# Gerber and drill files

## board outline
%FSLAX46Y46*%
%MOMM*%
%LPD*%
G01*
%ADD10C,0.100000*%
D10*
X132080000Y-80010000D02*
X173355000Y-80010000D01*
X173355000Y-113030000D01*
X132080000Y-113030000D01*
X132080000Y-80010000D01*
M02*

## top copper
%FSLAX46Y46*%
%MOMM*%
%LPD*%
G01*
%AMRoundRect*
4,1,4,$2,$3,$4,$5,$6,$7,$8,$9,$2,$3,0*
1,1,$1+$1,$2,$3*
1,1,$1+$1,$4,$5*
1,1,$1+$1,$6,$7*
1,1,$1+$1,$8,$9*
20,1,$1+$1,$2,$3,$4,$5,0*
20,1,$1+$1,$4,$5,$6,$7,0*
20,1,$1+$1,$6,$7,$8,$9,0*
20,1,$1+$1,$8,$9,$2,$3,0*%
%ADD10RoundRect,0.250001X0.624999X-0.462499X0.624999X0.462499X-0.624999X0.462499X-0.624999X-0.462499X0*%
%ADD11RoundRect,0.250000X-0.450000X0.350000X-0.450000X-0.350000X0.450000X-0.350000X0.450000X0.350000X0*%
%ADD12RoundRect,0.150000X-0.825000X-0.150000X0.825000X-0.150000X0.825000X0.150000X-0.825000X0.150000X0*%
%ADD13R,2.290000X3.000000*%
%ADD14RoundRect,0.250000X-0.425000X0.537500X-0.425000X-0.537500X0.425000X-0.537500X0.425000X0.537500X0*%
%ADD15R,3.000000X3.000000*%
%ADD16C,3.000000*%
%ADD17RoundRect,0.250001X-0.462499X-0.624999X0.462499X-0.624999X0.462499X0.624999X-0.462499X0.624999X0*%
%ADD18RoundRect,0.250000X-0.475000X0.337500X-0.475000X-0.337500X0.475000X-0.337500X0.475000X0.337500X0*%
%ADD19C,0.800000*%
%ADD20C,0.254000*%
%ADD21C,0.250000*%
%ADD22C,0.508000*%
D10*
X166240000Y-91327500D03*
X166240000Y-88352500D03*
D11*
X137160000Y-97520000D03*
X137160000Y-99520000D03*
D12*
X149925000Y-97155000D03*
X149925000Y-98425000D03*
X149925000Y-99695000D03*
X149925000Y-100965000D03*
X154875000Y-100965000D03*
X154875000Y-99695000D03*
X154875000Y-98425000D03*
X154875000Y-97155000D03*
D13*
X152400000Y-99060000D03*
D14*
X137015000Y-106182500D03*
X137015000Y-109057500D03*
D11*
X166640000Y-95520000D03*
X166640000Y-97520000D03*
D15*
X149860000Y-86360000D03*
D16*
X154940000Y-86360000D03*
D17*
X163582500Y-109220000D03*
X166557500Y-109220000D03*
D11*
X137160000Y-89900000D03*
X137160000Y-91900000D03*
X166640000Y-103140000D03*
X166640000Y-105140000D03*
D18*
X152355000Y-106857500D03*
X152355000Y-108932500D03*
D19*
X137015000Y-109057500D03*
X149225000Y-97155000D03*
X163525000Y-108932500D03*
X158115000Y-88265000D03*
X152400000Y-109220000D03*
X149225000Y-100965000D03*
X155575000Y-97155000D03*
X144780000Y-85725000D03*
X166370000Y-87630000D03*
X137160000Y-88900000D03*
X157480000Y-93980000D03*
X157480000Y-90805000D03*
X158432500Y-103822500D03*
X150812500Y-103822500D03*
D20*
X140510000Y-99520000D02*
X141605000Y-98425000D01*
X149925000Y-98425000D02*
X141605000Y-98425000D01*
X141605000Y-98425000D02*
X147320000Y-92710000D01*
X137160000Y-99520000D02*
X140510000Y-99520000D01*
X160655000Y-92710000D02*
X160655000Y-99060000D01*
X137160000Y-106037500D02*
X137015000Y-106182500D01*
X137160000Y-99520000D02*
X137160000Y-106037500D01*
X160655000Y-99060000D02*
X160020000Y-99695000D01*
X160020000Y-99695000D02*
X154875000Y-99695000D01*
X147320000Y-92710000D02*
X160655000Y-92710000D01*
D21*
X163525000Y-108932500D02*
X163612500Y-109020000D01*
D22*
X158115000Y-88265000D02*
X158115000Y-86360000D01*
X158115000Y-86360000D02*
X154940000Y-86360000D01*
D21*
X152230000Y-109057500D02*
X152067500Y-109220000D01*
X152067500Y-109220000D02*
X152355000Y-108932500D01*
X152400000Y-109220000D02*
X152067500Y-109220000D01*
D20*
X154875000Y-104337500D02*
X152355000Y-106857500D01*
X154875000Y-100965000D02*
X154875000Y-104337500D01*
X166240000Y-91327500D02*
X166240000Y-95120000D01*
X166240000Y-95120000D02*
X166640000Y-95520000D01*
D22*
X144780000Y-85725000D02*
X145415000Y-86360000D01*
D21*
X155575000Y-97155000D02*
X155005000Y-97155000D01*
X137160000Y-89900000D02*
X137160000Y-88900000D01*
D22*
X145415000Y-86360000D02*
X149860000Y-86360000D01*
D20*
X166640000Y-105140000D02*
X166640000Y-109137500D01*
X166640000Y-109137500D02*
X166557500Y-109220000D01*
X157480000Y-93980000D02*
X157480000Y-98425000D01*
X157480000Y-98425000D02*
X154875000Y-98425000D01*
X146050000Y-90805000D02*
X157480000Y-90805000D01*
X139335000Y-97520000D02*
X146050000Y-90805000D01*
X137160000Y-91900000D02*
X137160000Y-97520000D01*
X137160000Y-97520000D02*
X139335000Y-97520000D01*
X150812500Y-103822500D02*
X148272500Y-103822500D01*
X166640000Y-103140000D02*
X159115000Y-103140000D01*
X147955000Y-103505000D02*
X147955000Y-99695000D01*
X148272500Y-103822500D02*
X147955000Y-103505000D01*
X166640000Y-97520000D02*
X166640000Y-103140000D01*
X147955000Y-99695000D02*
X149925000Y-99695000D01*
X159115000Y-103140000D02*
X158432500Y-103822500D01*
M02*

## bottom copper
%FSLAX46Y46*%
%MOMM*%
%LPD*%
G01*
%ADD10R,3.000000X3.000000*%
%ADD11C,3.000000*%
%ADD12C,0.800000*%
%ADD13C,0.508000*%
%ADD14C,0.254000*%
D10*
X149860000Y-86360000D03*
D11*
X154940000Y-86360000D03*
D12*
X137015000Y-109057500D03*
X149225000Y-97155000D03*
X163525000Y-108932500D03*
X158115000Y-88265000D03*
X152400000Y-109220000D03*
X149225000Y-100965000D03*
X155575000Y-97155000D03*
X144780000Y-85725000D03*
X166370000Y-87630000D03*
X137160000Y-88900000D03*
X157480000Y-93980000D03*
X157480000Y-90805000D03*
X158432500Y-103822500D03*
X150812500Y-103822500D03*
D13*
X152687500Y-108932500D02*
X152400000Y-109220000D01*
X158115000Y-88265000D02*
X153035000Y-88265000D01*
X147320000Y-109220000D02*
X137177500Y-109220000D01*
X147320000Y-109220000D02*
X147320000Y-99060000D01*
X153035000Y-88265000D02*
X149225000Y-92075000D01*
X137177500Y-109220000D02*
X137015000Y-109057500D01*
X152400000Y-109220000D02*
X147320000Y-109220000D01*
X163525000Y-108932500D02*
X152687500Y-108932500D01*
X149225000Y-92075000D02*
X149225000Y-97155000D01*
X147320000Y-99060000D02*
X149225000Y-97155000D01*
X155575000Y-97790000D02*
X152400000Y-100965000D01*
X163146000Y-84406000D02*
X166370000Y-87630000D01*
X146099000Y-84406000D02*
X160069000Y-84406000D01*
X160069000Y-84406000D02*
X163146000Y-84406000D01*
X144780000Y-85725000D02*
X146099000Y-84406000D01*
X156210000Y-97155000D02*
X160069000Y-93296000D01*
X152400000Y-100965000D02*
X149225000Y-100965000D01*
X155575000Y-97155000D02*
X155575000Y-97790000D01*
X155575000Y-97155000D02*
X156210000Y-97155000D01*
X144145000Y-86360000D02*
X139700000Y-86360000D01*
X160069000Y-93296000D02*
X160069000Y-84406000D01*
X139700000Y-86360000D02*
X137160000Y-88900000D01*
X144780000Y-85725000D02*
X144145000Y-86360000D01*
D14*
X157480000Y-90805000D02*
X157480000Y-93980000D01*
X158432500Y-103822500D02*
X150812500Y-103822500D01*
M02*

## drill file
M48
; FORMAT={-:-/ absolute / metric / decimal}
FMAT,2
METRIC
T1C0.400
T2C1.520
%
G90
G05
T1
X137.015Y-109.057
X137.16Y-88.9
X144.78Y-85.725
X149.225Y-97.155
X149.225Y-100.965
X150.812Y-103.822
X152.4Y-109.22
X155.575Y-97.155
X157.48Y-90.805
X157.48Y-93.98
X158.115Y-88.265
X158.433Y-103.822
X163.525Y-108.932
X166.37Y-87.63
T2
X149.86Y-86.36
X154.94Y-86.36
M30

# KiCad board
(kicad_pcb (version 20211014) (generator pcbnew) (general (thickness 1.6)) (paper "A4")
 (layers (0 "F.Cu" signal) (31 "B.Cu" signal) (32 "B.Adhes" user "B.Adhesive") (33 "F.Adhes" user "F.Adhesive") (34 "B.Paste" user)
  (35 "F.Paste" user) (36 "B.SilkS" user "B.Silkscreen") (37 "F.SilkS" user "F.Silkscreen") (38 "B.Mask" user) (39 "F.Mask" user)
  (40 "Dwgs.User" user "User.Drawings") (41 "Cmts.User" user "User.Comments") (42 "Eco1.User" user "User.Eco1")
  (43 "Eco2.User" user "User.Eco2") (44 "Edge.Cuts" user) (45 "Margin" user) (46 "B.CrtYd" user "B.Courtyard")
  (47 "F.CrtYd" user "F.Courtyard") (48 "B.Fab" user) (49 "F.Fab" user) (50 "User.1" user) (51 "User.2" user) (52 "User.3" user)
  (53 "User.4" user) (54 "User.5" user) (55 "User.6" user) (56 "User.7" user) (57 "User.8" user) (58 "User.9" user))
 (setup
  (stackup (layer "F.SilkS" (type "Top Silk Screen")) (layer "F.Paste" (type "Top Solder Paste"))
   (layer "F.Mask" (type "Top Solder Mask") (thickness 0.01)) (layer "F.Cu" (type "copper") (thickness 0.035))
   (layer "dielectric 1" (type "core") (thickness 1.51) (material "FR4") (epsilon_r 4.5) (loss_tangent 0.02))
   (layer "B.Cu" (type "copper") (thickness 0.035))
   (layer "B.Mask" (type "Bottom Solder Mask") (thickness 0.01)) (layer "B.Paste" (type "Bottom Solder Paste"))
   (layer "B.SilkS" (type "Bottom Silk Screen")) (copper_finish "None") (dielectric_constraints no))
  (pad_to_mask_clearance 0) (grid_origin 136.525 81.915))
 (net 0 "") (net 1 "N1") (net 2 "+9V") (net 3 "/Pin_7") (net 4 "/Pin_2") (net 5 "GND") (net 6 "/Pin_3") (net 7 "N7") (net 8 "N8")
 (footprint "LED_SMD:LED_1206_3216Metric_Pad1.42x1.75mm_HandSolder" (layer "F.Cu") (at 166.24 89.84 90)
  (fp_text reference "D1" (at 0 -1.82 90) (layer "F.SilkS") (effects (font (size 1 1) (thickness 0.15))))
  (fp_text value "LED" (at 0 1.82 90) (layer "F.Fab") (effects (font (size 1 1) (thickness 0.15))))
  (pad "1" smd roundrect (at -1.4875 0 90) (size 1.425 1.75) (layers "F.Cu" "F.Paste" "F.Mask") (roundrect_rratio 0.1754392982) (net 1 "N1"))
  (pad "2" smd roundrect (at 1.4875 0 90) (size 1.425 1.75) (layers "F.Cu" "F.Paste" "F.Mask") (roundrect_rratio 0.1754392982) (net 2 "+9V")))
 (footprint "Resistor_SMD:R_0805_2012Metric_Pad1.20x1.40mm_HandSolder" (layer "F.Cu") (at 137.16 98.52 -90)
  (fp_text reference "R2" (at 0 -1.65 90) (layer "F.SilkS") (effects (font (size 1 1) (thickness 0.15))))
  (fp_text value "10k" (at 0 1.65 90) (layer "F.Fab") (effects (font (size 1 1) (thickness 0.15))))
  (pad "1" smd roundrect (at -1 0 270) (size 1.2 1.4) (layers "F.Cu" "F.Paste" "F.Mask") (roundrect_rratio 0.2083333333) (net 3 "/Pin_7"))
  (pad "2" smd roundrect (at 1 0 270) (size 1.2 1.4) (layers "F.Cu" "F.Paste" "F.Mask") (roundrect_rratio 0.2083333333) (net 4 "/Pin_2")))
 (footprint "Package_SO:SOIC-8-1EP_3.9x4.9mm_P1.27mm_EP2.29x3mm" (layer "F.Cu") (at 152.4 99.06)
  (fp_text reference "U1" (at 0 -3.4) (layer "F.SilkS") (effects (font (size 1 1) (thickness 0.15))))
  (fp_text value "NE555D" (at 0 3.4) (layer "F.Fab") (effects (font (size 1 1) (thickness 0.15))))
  (pad "" smd roundrect (at -0.57 -0.75) (size 0.92 1.21) (layers "F.Paste") (roundrect_rratio 0.25))
  (pad "" smd roundrect (at 0.57 0.75) (size 0.92 1.21) (layers "F.Paste") (roundrect_rratio 0.25))
  (pad "" smd roundrect (at -0.57 0.75) (size 0.92 1.21) (layers "F.Paste") (roundrect_rratio 0.25))
  (pad "" smd roundrect (at 0.57 -0.75) (size 0.92 1.21) (layers "F.Paste") (roundrect_rratio 0.25))
  (pad "1" smd roundrect (at -2.475 -1.905) (size 1.95 0.6) (layers "F.Cu" "F.Paste" "F.Mask") (roundrect_rratio 0.25) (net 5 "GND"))
  (pad "2" smd roundrect (at -2.475 -0.635) (size 1.95 0.6) (layers "F.Cu" "F.Paste" "F.Mask") (roundrect_rratio 0.25) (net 4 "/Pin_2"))
  (pad "3" smd roundrect (at -2.475 0.635) (size 1.95 0.6) (layers "F.Cu" "F.Paste" "F.Mask") (roundrect_rratio 0.25) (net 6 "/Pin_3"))
  (pad "4" smd roundrect (at -2.475 1.905) (size 1.95 0.6) (layers "F.Cu" "F.Paste" "F.Mask") (roundrect_rratio 0.25) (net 2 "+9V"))
  (pad "5" smd roundrect (at 2.475 1.905) (size 1.95 0.6) (layers "F.Cu" "F.Paste" "F.Mask") (roundrect_rratio 0.25) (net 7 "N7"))
  (pad "6" smd roundrect (at 2.475 0.635) (size 1.95 0.6) (layers "F.Cu" "F.Paste" "F.Mask") (roundrect_rratio 0.25) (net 4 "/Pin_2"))
  (pad "7" smd roundrect (at 2.475 -0.635) (size 1.95 0.6) (layers "F.Cu" "F.Paste" "F.Mask") (roundrect_rratio 0.25) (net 3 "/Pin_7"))
  (pad "8" smd roundrect (at 2.475 -1.905) (size 1.95 0.6) (layers "F.Cu" "F.Paste" "F.Mask") (roundrect_rratio 0.25) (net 2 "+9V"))
  (pad "9" smd rect (at 0 0) (size 2.29 3) (layers "F.Cu" "F.Mask")))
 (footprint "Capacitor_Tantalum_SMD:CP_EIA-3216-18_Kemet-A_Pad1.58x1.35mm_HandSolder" (layer "F.Cu") (at 137.015 107.62 -90)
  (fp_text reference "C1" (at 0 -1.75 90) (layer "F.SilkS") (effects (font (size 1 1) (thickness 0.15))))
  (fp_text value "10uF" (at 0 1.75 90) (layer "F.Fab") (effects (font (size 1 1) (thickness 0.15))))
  (pad "1" smd roundrect (at -1.4375 0 270) (size 1.575 1.35) (layers "F.Cu" "F.Paste" "F.Mask") (roundrect_rratio 0.1851851852)
   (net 4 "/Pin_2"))
  (pad "2" smd roundrect (at 1.4375 0 270) (size 1.575 1.35) (layers "F.Cu" "F.Paste" "F.Mask") (roundrect_rratio 0.1851851852)
   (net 5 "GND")))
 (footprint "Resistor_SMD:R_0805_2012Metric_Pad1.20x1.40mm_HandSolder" (layer "F.Cu") (at 166.64 96.52 -90)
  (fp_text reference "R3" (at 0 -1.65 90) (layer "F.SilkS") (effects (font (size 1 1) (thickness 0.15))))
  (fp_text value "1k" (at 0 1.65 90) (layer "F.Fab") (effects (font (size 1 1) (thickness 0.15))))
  (pad "1" smd roundrect (at -1 0 270) (size 1.2 1.4) (layers "F.Cu" "F.Paste" "F.Mask") (roundrect_rratio 0.2083333333) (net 1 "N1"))
  (pad "2" smd roundrect (at 1 0 270) (size 1.2 1.4) (layers "F.Cu" "F.Paste" "F.Mask") (roundrect_rratio 0.2083333333) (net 6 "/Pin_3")))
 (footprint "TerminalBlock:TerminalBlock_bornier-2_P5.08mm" (layer "F.Cu") (at 149.86 86.36)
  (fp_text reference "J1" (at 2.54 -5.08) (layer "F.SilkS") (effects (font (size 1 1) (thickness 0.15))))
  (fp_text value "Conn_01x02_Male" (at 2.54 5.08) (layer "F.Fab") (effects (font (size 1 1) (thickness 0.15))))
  (pad "1" thru_hole rect (at 0 0) (size 3 3) (drill 1.52) (layers *.Cu *.Mask) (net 2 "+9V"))
  (pad "2" thru_hole circle (at 5.08 0) (size 3 3) (drill 1.52) (layers *.Cu *.Mask) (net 5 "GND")))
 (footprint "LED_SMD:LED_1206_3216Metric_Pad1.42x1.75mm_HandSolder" (layer "F.Cu") (at 165.07 109.22)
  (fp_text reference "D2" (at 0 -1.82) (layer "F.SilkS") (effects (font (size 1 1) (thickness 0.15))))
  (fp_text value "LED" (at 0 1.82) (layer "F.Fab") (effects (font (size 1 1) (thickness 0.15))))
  (pad "1" smd roundrect (at -1.4875 0) (size 1.425 1.75) (layers "F.Cu" "F.Paste" "F.Mask") (roundrect_rratio 0.1754392982) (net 5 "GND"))
  (pad "2" smd roundrect (at 1.4875 0) (size 1.425 1.75) (layers "F.Cu" "F.Paste" "F.Mask") (roundrect_rratio 0.1754392982) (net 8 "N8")))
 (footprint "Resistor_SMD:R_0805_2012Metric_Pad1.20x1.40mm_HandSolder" (layer "F.Cu") (at 137.16 90.9 -90)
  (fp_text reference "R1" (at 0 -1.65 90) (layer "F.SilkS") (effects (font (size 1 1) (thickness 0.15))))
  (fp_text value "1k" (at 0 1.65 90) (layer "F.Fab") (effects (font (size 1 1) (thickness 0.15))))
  (pad "1" smd roundrect (at -1 0 270) (size 1.2 1.4) (layers "F.Cu" "F.Paste" "F.Mask") (roundrect_rratio 0.2083333333) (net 2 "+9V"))
  (pad "2" smd roundrect (at 1 0 270) (size 1.2 1.4) (layers "F.Cu" "F.Paste" "F.Mask") (roundrect_rratio 0.2083333333) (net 3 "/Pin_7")))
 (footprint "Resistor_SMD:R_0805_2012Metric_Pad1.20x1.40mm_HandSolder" (layer "F.Cu") (at 166.64 104.14 -90)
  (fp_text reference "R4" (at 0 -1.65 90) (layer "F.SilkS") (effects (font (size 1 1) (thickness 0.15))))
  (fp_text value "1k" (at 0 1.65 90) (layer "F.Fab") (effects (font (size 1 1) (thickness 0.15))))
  (pad "1" smd roundrect (at -1 0 270) (size 1.2 1.4) (layers "F.Cu" "F.Paste" "F.Mask") (roundrect_rratio 0.2083333333) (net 6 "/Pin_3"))
  (pad "2" smd roundrect (at 1 0 270) (size 1.2 1.4) (layers "F.Cu" "F.Paste" "F.Mask") (roundrect_rratio 0.2083333333) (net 8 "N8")))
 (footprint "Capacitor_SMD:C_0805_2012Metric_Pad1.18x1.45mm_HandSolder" (layer "F.Cu") (at 152.355 107.895 -90)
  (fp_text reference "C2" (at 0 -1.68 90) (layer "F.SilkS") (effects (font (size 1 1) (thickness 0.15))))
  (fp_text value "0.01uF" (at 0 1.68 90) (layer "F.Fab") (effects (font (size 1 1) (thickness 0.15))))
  (pad "1" smd roundrect (at -1.0375 0 270) (size 1.175 1.45) (layers "F.Cu" "F.Paste" "F.Mask") (roundrect_rratio 0.2127659574)
   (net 7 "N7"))
  (pad "2" smd roundrect (at 1.0375 0 270) (size 1.175 1.45) (layers "F.Cu" "F.Paste" "F.Mask") (roundrect_rratio 0.2127659574)
   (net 5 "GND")))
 (gr_rect (start 132.08 80.01) (end 173.355 113.03) (layer "Edge.Cuts") (width 0.1) (fill none))
 (segment (start 140.51 99.52) (end 141.605 98.425) (width 0.254) (layer "F.Cu") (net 4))
 (segment (start 149.925 98.425) (end 141.605 98.425) (width 0.254) (layer "F.Cu") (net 4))
 (segment (start 141.605 98.425) (end 147.32 92.71) (width 0.254) (layer "F.Cu") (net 4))
 (segment (start 137.16 99.52) (end 140.51 99.52) (width 0.254) (layer "F.Cu") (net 4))
 (segment (start 160.655 92.71) (end 160.655 99.06) (width 0.254) (layer "F.Cu") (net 4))
 (segment (start 137.16 106.0375) (end 137.015 106.1825) (width 0.254) (layer "F.Cu") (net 4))
 (segment (start 137.16 99.52) (end 137.16 106.0375) (width 0.254) (layer "F.Cu") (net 4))
 (segment (start 160.655 99.06) (end 160.02 99.695) (width 0.254) (layer "F.Cu") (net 4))
 (segment (start 160.02 99.695) (end 154.875 99.695) (width 0.254) (layer "F.Cu") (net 4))
 (segment (start 147.32 92.71) (end 160.655 92.71) (width 0.254) (layer "F.Cu") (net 4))
 (segment (start 163.525 108.9325) (end 163.6125 109.02) (width 0.25) (layer "F.Cu") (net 5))
 (segment (start 158.115 88.265) (end 158.115 86.36) (width 0.508) (layer "F.Cu") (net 5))
 (segment (start 158.115 86.36) (end 154.94 86.36) (width 0.508) (layer "F.Cu") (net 5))
 (segment (start 152.23 109.0575) (end 152.0675 109.22) (width 0.25) (layer "F.Cu") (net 5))
 (segment (start 152.0675 109.22) (end 152.355 108.9325) (width 0.25) (layer "F.Cu") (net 5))
 (segment (start 152.4 109.22) (end 152.0675 109.22) (width 0.25) (layer "F.Cu") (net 5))
 (via (at 137.015 109.0575) (size 0.8) (drill 0.4) (layers "F.Cu" "B.Cu") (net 5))
 (via (at 149.225 97.155) (size 0.8) (drill 0.4) (layers "F.Cu" "B.Cu") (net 5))
 (via (at 163.525 108.9325) (size 0.8) (drill 0.4) (layers "F.Cu" "B.Cu") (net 5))
 (via (at 158.115 88.265) (size 0.8) (drill 0.4) (layers "F.Cu" "B.Cu") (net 5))
 (via (at 152.4 109.22) (size 0.8) (drill 0.4) (layers "F.Cu" "B.Cu") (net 5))
 (segment (start 152.6875 108.9325) (end 152.4 109.22) (width 0.508) (layer "B.Cu") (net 5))
 (segment (start 158.115 88.265) (end 153.035 88.265) (width 0.508) (layer "B.Cu") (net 5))
 (segment (start 147.32 109.22) (end 137.1775 109.22) (width 0.508) (layer "B.Cu") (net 5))
 (segment (start 147.32 109.22) (end 147.32 99.06) (width 0.508) (layer "B.Cu") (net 5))
 (segment (start 153.035 88.265) (end 149.225 92.075) (width 0.508) (layer "B.Cu") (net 5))
 (segment (start 137.1775 109.22) (end 137.015 109.0575) (width 0.508) (layer "B.Cu") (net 5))
 (segment (start 152.4 109.22) (end 147.32 109.22) (width 0.508) (layer "B.Cu") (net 5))
 (segment (start 163.525 108.9325) (end 152.6875 108.9325) (width 0.508) (layer "B.Cu") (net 5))
 (segment (start 149.225 92.075) (end 149.225 97.155) (width 0.508) (layer "B.Cu") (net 5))
 (segment (start 147.32 99.06) (end 149.225 97.155) (width 0.508) (layer "B.Cu") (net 5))
 (segment (start 154.875 104.3375) (end 152.355 106.8575) (width 0.254) (layer "F.Cu") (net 7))
 (segment (start 154.875 100.965) (end 154.875 104.3375) (width 0.254) (layer "F.Cu") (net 7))
 (segment (start 166.24 91.3275) (end 166.24 95.12) (width 0.254) (layer "F.Cu") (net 1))
 (segment (start 166.24 95.12) (end 166.64 95.52) (width 0.254) (layer "F.Cu") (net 1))
 (segment (start 144.78 85.725) (end 145.415 86.36) (width 0.508) (layer "F.Cu") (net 2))
 (segment (start 155.575 97.155) (end 155.005 97.155) (width 0.25) (layer "F.Cu") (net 2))
 (segment (start 137.16 89.9) (end 137.16 88.9) (width 0.25) (layer "F.Cu") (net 2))
 (segment (start 145.415 86.36) (end 149.86 86.36) (width 0.508) (layer "F.Cu") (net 2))
 (via (at 149.225 100.965) (size 0.8) (drill 0.4) (layers "F.Cu" "B.Cu") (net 2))
 (via (at 155.575 97.155) (size 0.8) (drill 0.4) (layers "F.Cu" "B.Cu") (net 2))
 (via (at 144.78 85.725) (size 0.8) (drill 0.4) (layers "F.Cu" "B.Cu") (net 2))
 (via (at 166.37 87.63) (size 0.8) (drill 0.4) (layers "F.Cu" "B.Cu") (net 2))
 (via (at 137.16 88.9) (size 0.8) (drill 0.4) (layers "F.Cu" "B.Cu") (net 2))
 (segment (start 155.575 97.79) (end 152.4 100.965) (width 0.508) (layer "B.Cu") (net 2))
 (segment (start 163.146 84.406) (end 166.37 87.63) (width 0.508) (layer "B.Cu") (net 2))
 (segment (start 146.099 84.406) (end 160.069 84.406) (width 0.508) (layer "B.Cu") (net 2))
 (segment (start 160.069 84.406) (end 163.146 84.406) (width 0.508) (layer "B.Cu") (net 2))
 (segment (start 144.78 85.725) (end 146.099 84.406) (width 0.508) (layer "B.Cu") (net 2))
 (segment (start 156.21 97.155) (end 160.069 93.296) (width 0.508) (layer "B.Cu") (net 2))
 (segment (start 152.4 100.965) (end 149.225 100.965) (width 0.508) (layer "B.Cu") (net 2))
 (segment (start 155.575 97.155) (end 155.575 97.79) (width 0.508) (layer "B.Cu") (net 2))
 (segment (start 155.575 97.155) (end 156.21 97.155) (width 0.508) (layer "B.Cu") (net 2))
 (segment (start 144.145 86.36) (end 139.7 86.36) (width 0.508) (layer "B.Cu") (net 2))
 (segment (start 160.069 93.296) (end 160.069 84.406) (width 0.508) (layer "B.Cu") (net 2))
 (segment (start 139.7 86.36) (end 137.16 88.9) (width 0.508) (layer "B.Cu") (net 2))
 (segment (start 144.78 85.725) (end 144.145 86.36) (width 0.508) (layer "B.Cu") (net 2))
 (segment (start 166.64 105.14) (end 166.64 109.1375) (width 0.254) (layer "F.Cu") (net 8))
 (segment (start 166.64 109.1375) (end 166.5575 109.22) (width 0.254) (layer "F.Cu") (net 8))
 (segment (start 157.48 93.98) (end 157.48 98.425) (width 0.254) (layer "F.Cu") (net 3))
 (segment (start 157.48 98.425) (end 154.875 98.425) (width 0.254) (layer "F.Cu") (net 3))
 (segment (start 146.05 90.805) (end 157.48 90.805) (width 0.254) (layer "F.Cu") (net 3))
 (segment (start 139.335 97.52) (end 146.05 90.805) (width 0.254) (layer "F.Cu") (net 3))
 (segment (start 137.16 91.9) (end 137.16 97.52) (width 0.254) (layer "F.Cu") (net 3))
 (segment (start 137.16 97.52) (end 139.335 97.52) (width 0.254) (layer "F.Cu") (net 3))
 (via (at 157.48 93.98) (size 0.8) (drill 0.4) (layers "F.Cu" "B.Cu") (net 3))
 (via (at 157.48 90.805) (size 0.8) (drill 0.4) (layers "F.Cu" "B.Cu") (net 3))
 (segment (start 157.48 90.805) (end 157.48 93.98) (width 0.254) (layer "B.Cu") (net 3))
 (segment (start 150.8125 103.8225) (end 148.2725 103.8225) (width 0.254) (layer "F.Cu") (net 6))
 (segment (start 166.64 103.14) (end 159.115 103.14) (width 0.254) (layer "F.Cu") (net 6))
 (segment (start 147.955 103.505) (end 147.955 99.695) (width 0.254) (layer "F.Cu") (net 6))
 (segment (start 148.2725 103.8225) (end 147.955 103.505) (width 0.254) (layer "F.Cu") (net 6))
 (segment (start 166.64 97.52) (end 166.64 103.14) (width 0.254) (layer "F.Cu") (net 6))
 (segment (start 147.955 99.695) (end 149.925 99.695) (width 0.254) (layer "F.Cu") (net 6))
 (segment (start 159.115 103.14) (end 158.4325 103.8225) (width 0.254) (layer "F.Cu") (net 6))
 (via (at 158.4325 103.8225) (size 0.8) (drill 0.4) (layers "F.Cu" "B.Cu") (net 6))
 (via (at 150.8125 103.8225) (size 0.8) (drill 0.4) (layers "F.Cu" "B.Cu") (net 6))
 (segment (start 158.4325 103.8225) (end 150.8125 103.8225) (width 0.254) (layer "B.Cu") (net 6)))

